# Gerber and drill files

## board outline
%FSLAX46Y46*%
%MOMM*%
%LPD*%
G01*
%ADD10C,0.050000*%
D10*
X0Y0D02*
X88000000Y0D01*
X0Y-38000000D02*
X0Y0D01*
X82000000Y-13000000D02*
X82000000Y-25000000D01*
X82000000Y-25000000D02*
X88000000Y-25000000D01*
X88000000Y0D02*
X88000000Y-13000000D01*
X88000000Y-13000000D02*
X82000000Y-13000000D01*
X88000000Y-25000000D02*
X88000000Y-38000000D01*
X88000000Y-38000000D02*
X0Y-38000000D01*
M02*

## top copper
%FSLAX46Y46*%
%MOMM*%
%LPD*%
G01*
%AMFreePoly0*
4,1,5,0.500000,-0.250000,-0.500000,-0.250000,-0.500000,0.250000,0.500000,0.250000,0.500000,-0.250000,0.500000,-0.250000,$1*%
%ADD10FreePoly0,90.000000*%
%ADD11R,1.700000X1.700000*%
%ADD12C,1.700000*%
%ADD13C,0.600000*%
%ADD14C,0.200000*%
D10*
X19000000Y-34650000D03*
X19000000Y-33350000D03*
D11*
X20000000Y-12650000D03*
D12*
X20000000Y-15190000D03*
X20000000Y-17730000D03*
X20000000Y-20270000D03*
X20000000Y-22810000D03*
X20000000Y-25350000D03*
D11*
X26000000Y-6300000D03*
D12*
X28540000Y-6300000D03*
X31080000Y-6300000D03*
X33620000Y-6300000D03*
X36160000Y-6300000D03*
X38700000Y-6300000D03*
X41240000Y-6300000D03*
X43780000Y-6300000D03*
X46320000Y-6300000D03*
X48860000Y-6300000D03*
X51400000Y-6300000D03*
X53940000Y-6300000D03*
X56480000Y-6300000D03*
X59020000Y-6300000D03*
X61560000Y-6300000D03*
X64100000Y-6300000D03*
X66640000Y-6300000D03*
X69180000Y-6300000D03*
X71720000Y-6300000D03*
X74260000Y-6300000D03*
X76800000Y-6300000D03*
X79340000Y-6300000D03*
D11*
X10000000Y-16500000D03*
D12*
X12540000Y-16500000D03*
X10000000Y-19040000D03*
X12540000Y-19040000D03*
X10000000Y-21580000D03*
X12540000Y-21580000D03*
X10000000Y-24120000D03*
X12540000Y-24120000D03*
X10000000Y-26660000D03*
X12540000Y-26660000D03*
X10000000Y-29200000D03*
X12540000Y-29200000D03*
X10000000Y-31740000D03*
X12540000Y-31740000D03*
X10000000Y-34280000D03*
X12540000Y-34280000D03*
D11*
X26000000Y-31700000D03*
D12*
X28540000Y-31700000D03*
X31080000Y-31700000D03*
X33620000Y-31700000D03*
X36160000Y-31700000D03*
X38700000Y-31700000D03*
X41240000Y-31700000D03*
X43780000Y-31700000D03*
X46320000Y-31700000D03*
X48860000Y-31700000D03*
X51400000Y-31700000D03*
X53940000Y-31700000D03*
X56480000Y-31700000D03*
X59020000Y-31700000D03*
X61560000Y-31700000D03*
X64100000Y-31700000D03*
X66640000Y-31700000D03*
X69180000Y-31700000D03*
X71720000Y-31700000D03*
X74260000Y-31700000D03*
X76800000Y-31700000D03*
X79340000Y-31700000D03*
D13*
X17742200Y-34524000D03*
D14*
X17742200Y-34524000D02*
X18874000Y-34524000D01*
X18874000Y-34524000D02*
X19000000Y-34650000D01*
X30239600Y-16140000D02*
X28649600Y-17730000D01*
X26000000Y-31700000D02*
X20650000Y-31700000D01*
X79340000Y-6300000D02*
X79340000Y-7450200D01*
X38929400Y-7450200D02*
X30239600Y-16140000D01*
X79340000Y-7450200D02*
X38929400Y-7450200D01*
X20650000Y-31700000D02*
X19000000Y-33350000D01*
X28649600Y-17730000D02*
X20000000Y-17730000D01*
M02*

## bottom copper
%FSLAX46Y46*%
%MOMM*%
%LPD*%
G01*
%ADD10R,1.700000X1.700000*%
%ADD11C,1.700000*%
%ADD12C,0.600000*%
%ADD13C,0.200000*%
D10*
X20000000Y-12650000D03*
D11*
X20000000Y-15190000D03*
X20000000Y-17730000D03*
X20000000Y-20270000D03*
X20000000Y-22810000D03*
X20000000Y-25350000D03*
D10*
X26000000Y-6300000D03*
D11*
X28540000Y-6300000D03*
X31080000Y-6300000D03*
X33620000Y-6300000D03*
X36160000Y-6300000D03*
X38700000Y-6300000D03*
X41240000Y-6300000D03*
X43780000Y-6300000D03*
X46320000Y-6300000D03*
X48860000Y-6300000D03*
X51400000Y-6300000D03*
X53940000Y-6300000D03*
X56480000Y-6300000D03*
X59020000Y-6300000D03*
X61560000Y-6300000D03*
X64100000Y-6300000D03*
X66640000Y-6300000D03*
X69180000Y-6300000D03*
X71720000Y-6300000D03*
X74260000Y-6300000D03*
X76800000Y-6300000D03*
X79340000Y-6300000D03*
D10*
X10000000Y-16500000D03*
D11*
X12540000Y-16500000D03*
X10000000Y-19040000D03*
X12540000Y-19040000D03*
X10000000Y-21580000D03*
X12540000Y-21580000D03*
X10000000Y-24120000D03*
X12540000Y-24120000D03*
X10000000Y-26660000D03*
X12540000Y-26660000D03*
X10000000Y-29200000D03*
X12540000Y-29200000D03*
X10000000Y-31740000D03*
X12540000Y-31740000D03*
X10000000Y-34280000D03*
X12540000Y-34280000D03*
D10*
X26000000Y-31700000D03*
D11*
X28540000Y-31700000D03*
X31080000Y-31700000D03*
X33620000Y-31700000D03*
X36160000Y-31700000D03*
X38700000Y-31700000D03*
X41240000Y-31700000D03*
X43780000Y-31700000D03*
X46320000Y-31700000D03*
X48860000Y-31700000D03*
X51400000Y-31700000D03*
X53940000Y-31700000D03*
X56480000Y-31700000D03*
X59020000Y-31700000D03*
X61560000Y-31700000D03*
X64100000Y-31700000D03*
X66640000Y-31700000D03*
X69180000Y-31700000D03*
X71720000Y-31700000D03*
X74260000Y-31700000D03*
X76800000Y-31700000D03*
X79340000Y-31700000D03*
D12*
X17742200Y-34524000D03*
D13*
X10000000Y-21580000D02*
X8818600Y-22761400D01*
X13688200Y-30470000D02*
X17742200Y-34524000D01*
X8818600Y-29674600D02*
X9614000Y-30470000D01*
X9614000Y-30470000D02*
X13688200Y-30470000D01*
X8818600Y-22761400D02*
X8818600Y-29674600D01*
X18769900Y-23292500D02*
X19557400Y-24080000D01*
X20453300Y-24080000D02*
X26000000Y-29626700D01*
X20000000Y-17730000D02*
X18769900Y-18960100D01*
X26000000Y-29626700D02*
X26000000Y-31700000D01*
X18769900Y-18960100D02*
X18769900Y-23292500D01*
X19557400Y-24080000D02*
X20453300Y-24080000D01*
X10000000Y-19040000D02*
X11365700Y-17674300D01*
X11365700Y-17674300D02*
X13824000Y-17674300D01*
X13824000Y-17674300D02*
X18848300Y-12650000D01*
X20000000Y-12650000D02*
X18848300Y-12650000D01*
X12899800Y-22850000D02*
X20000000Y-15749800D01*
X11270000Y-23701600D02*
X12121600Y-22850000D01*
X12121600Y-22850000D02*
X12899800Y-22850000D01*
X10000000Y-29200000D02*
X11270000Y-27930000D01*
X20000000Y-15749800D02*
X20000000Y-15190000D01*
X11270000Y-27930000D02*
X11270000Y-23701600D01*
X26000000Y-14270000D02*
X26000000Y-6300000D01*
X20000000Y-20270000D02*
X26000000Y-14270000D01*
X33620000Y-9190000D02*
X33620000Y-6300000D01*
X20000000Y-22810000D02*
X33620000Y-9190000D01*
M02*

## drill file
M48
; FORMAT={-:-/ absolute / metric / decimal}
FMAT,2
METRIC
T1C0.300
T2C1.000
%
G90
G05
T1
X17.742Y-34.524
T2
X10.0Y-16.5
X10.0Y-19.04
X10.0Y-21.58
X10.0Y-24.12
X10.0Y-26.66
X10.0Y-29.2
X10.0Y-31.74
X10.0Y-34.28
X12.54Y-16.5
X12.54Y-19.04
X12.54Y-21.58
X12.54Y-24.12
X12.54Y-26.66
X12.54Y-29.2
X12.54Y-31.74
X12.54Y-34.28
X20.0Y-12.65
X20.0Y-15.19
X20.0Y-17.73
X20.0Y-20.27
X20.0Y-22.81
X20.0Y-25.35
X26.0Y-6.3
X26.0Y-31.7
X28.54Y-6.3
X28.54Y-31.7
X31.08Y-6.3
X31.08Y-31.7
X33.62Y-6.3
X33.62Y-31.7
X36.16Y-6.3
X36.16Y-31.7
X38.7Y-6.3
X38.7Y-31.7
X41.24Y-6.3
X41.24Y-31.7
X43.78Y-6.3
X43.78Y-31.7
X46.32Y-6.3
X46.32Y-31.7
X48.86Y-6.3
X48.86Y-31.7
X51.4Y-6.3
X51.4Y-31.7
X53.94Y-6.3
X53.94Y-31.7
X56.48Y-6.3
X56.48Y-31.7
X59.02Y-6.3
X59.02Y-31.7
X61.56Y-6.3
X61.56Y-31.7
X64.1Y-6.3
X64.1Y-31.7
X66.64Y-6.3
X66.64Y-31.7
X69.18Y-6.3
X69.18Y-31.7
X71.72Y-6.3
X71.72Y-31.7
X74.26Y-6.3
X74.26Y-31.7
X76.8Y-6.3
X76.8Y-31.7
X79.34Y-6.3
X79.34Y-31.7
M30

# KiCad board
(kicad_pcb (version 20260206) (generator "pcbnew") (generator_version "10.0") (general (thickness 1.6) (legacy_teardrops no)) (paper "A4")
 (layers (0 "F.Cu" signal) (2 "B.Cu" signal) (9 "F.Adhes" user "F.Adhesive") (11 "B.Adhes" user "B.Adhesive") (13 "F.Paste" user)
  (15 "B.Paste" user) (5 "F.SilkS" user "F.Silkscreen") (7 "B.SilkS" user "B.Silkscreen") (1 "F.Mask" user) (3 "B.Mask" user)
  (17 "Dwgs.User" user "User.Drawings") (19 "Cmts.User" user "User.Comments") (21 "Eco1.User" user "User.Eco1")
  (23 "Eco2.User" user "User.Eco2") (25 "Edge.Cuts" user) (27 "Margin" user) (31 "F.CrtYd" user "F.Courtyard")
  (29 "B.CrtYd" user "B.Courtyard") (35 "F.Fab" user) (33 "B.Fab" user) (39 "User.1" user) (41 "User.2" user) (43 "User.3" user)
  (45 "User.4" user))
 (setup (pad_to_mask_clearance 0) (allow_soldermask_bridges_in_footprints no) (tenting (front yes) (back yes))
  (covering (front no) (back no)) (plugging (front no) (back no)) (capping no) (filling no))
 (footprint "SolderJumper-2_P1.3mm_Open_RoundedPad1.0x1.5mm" (layer "F.Cu") (at 19 34 90)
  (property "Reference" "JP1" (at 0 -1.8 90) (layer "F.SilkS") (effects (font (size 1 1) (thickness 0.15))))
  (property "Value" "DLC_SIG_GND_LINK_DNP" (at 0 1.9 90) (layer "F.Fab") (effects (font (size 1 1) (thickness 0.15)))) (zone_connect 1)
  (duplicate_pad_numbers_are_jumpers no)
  (pad "1" smd custom (at -0.65 0 90) (size 1 0.5) (layers "F.Cu" "F.Mask") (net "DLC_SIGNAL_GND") (zone_connect 2)
   (thermal_bridge_angle 45) (options (clearance outline) (anchor rect)) (primitives))
  (pad "2" smd custom (at 0.65 0 90) (size 1 0.5) (layers "F.Cu" "F.Mask") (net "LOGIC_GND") (zone_connect 2) (thermal_bridge_angle 45)
   (options (clearance outline) (anchor rect)) (primitives)))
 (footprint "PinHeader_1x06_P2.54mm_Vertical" (layer "F.Cu") (at 20 12.65)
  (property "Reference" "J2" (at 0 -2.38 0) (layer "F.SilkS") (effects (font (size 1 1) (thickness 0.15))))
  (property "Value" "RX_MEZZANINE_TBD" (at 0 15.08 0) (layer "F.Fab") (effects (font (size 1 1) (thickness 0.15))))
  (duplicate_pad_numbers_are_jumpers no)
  (pad "1" thru_hole rect (at 0 0) (size 1.7 1.7) (drill 1) (layers "*.Cu" "*.Mask") (remove_unused_layers no) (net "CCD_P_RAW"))
  (pad "2" thru_hole circle (at 0 2.54) (size 1.7 1.7) (drill 1) (layers "*.Cu" "*.Mask") (remove_unused_layers no) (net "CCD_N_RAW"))
  (pad "3" thru_hole circle (at 0 5.08) (size 1.7 1.7) (drill 1) (layers "*.Cu" "*.Mask") (remove_unused_layers no) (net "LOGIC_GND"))
  (pad "4" thru_hole circle (at 0 7.62) (size 1.7 1.7) (drill 1) (layers "*.Cu" "*.Mask") (remove_unused_layers no) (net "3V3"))
  (pad "5" thru_hole circle (at 0 10.16) (size 1.7 1.7) (drill 1) (layers "*.Cu" "*.Mask") (remove_unused_layers no) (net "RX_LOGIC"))
  (pad "6" thru_hole circle (at 0 12.7) (size 1.7 1.7) (drill 1) (layers "*.Cu" "*.Mask") (remove_unused_layers no)))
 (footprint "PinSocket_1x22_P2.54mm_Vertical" (layer "F.Cu") (at 26 6.3 90)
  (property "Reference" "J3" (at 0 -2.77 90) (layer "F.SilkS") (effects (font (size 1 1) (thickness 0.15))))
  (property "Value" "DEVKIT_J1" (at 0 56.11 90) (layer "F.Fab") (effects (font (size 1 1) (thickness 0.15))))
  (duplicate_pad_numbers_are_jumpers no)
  (pad "1" thru_hole rect (at 0 0 90) (size 1.7 1.7) (drill 1) (layers "*.Cu" "*.Mask") (remove_unused_layers no) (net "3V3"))
  (pad "2" thru_hole circle (at 0 2.54 90) (size 1.7 1.7) (drill 1) (layers "*.Cu" "*.Mask") (remove_unused_layers no))
  (pad "3" thru_hole circle (at 0 5.08 90) (size 1.7 1.7) (drill 1) (layers "*.Cu" "*.Mask") (remove_unused_layers no))
  (pad "4" thru_hole circle (at 0 7.62 90) (size 1.7 1.7) (drill 1) (layers "*.Cu" "*.Mask") (remove_unused_layers no) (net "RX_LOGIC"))
  (pad "5" thru_hole circle (at 0 10.16 90) (size 1.7 1.7) (drill 1) (layers "*.Cu" "*.Mask") (remove_unused_layers no))
  (pad "6" thru_hole circle (at 0 12.7 90) (size 1.7 1.7) (drill 1) (layers "*.Cu" "*.Mask") (remove_unused_layers no))
  (pad "7" thru_hole circle (at 0 15.24 90) (size 1.7 1.7) (drill 1) (layers "*.Cu" "*.Mask") (remove_unused_layers no))
  (pad "8" thru_hole circle (at 0 17.78 90) (size 1.7 1.7) (drill 1) (layers "*.Cu" "*.Mask") (remove_unused_layers no))
  (pad "9" thru_hole circle (at 0 20.32 90) (size 1.7 1.7) (drill 1) (layers "*.Cu" "*.Mask") (remove_unused_layers no))
  (pad "10" thru_hole circle (at 0 22.86 90) (size 1.7 1.7) (drill 1) (layers "*.Cu" "*.Mask") (remove_unused_layers no))
  (pad "11" thru_hole circle (at 0 25.4 90) (size 1.7 1.7) (drill 1) (layers "*.Cu" "*.Mask") (remove_unused_layers no))
  (pad "12" thru_hole circle (at 0 27.94 90) (size 1.7 1.7) (drill 1) (layers "*.Cu" "*.Mask") (remove_unused_layers no))
  (pad "13" thru_hole circle (at 0 30.48 90) (size 1.7 1.7) (drill 1) (layers "*.Cu" "*.Mask") (remove_unused_layers no))
  (pad "14" thru_hole circle (at 0 33.02 90) (size 1.7 1.7) (drill 1) (layers "*.Cu" "*.Mask") (remove_unused_layers no))
  (pad "15" thru_hole circle (at 0 35.56 90) (size 1.7 1.7) (drill 1) (layers "*.Cu" "*.Mask") (remove_unused_layers no))
  (pad "16" thru_hole circle (at 0 38.1 90) (size 1.7 1.7) (drill 1) (layers "*.Cu" "*.Mask") (remove_unused_layers no))
  (pad "17" thru_hole circle (at 0 40.64 90) (size 1.7 1.7) (drill 1) (layers "*.Cu" "*.Mask") (remove_unused_layers no))
  (pad "18" thru_hole circle (at 0 43.18 90) (size 1.7 1.7) (drill 1) (layers "*.Cu" "*.Mask") (remove_unused_layers no))
  (pad "19" thru_hole circle (at 0 45.72 90) (size 1.7 1.7) (drill 1) (layers "*.Cu" "*.Mask") (remove_unused_layers no))
  (pad "20" thru_hole circle (at 0 48.26 90) (size 1.7 1.7) (drill 1) (layers "*.Cu" "*.Mask") (remove_unused_layers no))
  (pad "21" thru_hole circle (at 0 50.8 90) (size 1.7 1.7) (drill 1) (layers "*.Cu" "*.Mask") (remove_unused_layers no))
  (pad "22" thru_hole circle (at 0 53.34 90) (size 1.7 1.7) (drill 1) (layers "*.Cu" "*.Mask") (remove_unused_layers no) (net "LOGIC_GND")))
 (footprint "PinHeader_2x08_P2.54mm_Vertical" (layer "F.Cu") (at 10 16.5)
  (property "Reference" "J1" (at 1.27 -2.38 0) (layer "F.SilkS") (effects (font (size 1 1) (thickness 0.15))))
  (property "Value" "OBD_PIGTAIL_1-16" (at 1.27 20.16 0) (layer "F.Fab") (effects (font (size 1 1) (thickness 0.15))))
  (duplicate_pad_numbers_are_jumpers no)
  (pad "1" thru_hole rect (at 0 0) (size 1.7 1.7) (drill 1) (layers "*.Cu" "*.Mask") (remove_unused_layers no))
  (pad "2" thru_hole circle (at 2.54 0) (size 1.7 1.7) (drill 1) (layers "*.Cu" "*.Mask") (remove_unused_layers no))
  (pad "3" thru_hole circle (at 0 2.54) (size 1.7 1.7) (drill 1) (layers "*.Cu" "*.Mask") (remove_unused_layers no) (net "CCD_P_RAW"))
  (pad "4" thru_hole circle (at 2.54 2.54) (size 1.7 1.7) (drill 1) (layers "*.Cu" "*.Mask") (remove_unused_layers no)
   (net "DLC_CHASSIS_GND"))
  (pad "5" thru_hole circle (at 0 5.08) (size 1.7 1.7) (drill 1) (layers "*.Cu" "*.Mask") (remove_unused_layers no) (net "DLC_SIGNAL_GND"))
  (pad "6" thru_hole circle (at 2.54 5.08) (size 1.7 1.7) (drill 1) (layers "*.Cu" "*.Mask") (remove_unused_layers no))
  (pad "7" thru_hole circle (at 0 7.62) (size 1.7 1.7) (drill 1) (layers "*.Cu" "*.Mask") (remove_unused_layers no))
  (pad "8" thru_hole circle (at 2.54 7.62) (size 1.7 1.7) (drill 1) (layers "*.Cu" "*.Mask") (remove_unused_layers no))
  (pad "9" thru_hole circle (at 0 10.16) (size 1.7 1.7) (drill 1) (layers "*.Cu" "*.Mask") (remove_unused_layers no))
  (pad "10" thru_hole circle (at 2.54 10.16) (size 1.7 1.7) (drill 1) (layers "*.Cu" "*.Mask") (remove_unused_layers no))
  (pad "11" thru_hole circle (at 0 12.7) (size 1.7 1.7) (drill 1) (layers "*.Cu" "*.Mask") (remove_unused_layers no) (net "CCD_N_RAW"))
  (pad "12" thru_hole circle (at 2.54 12.7) (size 1.7 1.7) (drill 1) (layers "*.Cu" "*.Mask") (remove_unused_layers no))
  (pad "13" thru_hole circle (at 0 15.24) (size 1.7 1.7) (drill 1) (layers "*.Cu" "*.Mask") (remove_unused_layers no))
  (pad "14" thru_hole circle (at 2.54 15.24) (size 1.7 1.7) (drill 1) (layers "*.Cu" "*.Mask") (remove_unused_layers no))
  (pad "15" thru_hole circle (at 0 17.78) (size 1.7 1.7) (drill 1) (layers "*.Cu" "*.Mask") (remove_unused_layers no))
  (pad "16" thru_hole circle (at 2.54 17.78) (size 1.7 1.7) (drill 1) (layers "*.Cu" "*.Mask") (remove_unused_layers no)))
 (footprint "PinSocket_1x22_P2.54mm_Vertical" (layer "F.Cu") (at 26 31.7 90)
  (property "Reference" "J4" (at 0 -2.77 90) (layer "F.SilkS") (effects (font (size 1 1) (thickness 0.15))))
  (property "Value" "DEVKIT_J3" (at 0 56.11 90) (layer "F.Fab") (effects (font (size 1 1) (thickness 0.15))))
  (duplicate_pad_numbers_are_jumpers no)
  (pad "1" thru_hole rect (at 0 0 90) (size 1.7 1.7) (drill 1) (layers "*.Cu" "*.Mask") (remove_unused_layers no) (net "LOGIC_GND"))
  (pad "2" thru_hole circle (at 0 2.54 90) (size 1.7 1.7) (drill 1) (layers "*.Cu" "*.Mask") (remove_unused_layers no))
  (pad "3" thru_hole circle (at 0 5.08 90) (size 1.7 1.7) (drill 1) (layers "*.Cu" "*.Mask") (remove_unused_layers no))
  (pad "4" thru_hole circle (at 0 7.62 90) (size 1.7 1.7) (drill 1) (layers "*.Cu" "*.Mask") (remove_unused_layers no))
  (pad "5" thru_hole circle (at 0 10.16 90) (size 1.7 1.7) (drill 1) (layers "*.Cu" "*.Mask") (remove_unused_layers no))
  (pad "6" thru_hole circle (at 0 12.7 90) (size 1.7 1.7) (drill 1) (layers "*.Cu" "*.Mask") (remove_unused_layers no))
  (pad "7" thru_hole circle (at 0 15.24 90) (size 1.7 1.7) (drill 1) (layers "*.Cu" "*.Mask") (remove_unused_layers no))
  (pad "8" thru_hole circle (at 0 17.78 90) (size 1.7 1.7) (drill 1) (layers "*.Cu" "*.Mask") (remove_unused_layers no))
  (pad "9" thru_hole circle (at 0 20.32 90) (size 1.7 1.7) (drill 1) (layers "*.Cu" "*.Mask") (remove_unused_layers no))
  (pad "10" thru_hole circle (at 0 22.86 90) (size 1.7 1.7) (drill 1) (layers "*.Cu" "*.Mask") (remove_unused_layers no))
  (pad "11" thru_hole circle (at 0 25.4 90) (size 1.7 1.7) (drill 1) (layers "*.Cu" "*.Mask") (remove_unused_layers no))
  (pad "12" thru_hole circle (at 0 27.94 90) (size 1.7 1.7) (drill 1) (layers "*.Cu" "*.Mask") (remove_unused_layers no))
  (pad "13" thru_hole circle (at 0 30.48 90) (size 1.7 1.7) (drill 1) (layers "*.Cu" "*.Mask") (remove_unused_layers no))
  (pad "14" thru_hole circle (at 0 33.02 90) (size 1.7 1.7) (drill 1) (layers "*.Cu" "*.Mask") (remove_unused_layers no))
  (pad "15" thru_hole circle (at 0 35.56 90) (size 1.7 1.7) (drill 1) (layers "*.Cu" "*.Mask") (remove_unused_layers no))
  (pad "16" thru_hole circle (at 0 38.1 90) (size 1.7 1.7) (drill 1) (layers "*.Cu" "*.Mask") (remove_unused_layers no))
  (pad "17" thru_hole circle (at 0 40.64 90) (size 1.7 1.7) (drill 1) (layers "*.Cu" "*.Mask") (remove_unused_layers no))
  (pad "18" thru_hole circle (at 0 43.18 90) (size 1.7 1.7) (drill 1) (layers "*.Cu" "*.Mask") (remove_unused_layers no))
  (pad "19" thru_hole circle (at 0 45.72 90) (size 1.7 1.7) (drill 1) (layers "*.Cu" "*.Mask") (remove_unused_layers no))
  (pad "20" thru_hole circle (at 0 48.26 90) (size 1.7 1.7) (drill 1) (layers "*.Cu" "*.Mask") (remove_unused_layers no))
  (pad "21" thru_hole circle (at 0 50.8 90) (size 1.7 1.7) (drill 1) (layers "*.Cu" "*.Mask") (remove_unused_layers no))
  (pad "22" thru_hole circle (at 0 53.34 90) (size 1.7 1.7) (drill 1) (layers "*.Cu" "*.Mask") (remove_unused_layers no)))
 (gr_line (start 0 0) (end 88 0) (stroke (width 0.05) (type default)) (layer "Edge.Cuts"))
 (gr_line (start 0 38) (end 0 0) (stroke (width 0.05) (type default)) (layer "Edge.Cuts"))
 (gr_line (start 82 13) (end 82 25) (stroke (width 0.05) (type default)) (layer "Edge.Cuts"))
 (gr_line (start 82 25) (end 88 25) (stroke (width 0.05) (type default)) (layer "Edge.Cuts"))
 (gr_line (start 88 0) (end 88 13) (stroke (width 0.05) (type default)) (layer "Edge.Cuts"))
 (gr_line (start 88 13) (end 82 13) (stroke (width 0.05) (type default)) (layer "Edge.Cuts"))
 (gr_line (start 88 25) (end 88 38) (stroke (width 0.05) (type default)) (layer "Edge.Cuts"))
 (gr_line (start 88 38) (end 0 38) (stroke (width 0.05) (type default)) (layer "Edge.Cuts"))
 (segment (start 17.7422 34.524) (end 18.874 34.524) (width 0.2) (layer "F.Cu") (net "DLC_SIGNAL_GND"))
 (segment (start 18.874 34.524) (end 19 34.65) (width 0.2) (layer "F.Cu") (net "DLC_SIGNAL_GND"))
 (via (at 17.7422 34.524) (size 0.6) (drill 0.3) (layers "F.Cu" "B.Cu") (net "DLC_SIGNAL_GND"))
 (segment (start 10 21.58) (end 8.8186 22.7614) (width 0.2) (layer "B.Cu") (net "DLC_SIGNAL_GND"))
 (segment (start 13.6882 30.47) (end 17.7422 34.524) (width 0.2) (layer "B.Cu") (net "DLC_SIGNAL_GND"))
 (segment (start 8.8186 29.6746) (end 9.614 30.47) (width 0.2) (layer "B.Cu") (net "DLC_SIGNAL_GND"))
 (segment (start 9.614 30.47) (end 13.6882 30.47) (width 0.2) (layer "B.Cu") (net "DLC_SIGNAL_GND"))
 (segment (start 8.8186 22.7614) (end 8.8186 29.6746) (width 0.2) (layer "B.Cu") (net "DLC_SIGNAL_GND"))
 (segment (start 30.2396 16.14) (end 28.6496 17.73) (width 0.2) (layer "F.Cu") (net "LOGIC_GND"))
 (segment (start 26 31.7) (end 20.65 31.7) (width 0.2) (layer "F.Cu") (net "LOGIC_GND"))
 (segment (start 79.34 6.3) (end 79.34 7.4502) (width 0.2) (layer "F.Cu") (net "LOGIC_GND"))
 (segment (start 38.9294 7.4502) (end 30.2396 16.14) (width 0.2) (layer "F.Cu") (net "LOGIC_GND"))
 (segment (start 79.34 7.4502) (end 38.9294 7.4502) (width 0.2) (layer "F.Cu") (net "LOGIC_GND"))
 (segment (start 20.65 31.7) (end 19 33.35) (width 0.2) (layer "F.Cu") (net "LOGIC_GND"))
 (segment (start 28.6496 17.73) (end 20 17.73) (width 0.2) (layer "F.Cu") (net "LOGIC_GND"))
 (segment (start 18.7699 23.2925) (end 19.5574 24.08) (width 0.2) (layer "B.Cu") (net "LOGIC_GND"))
 (segment (start 20.4533 24.08) (end 26 29.6267) (width 0.2) (layer "B.Cu") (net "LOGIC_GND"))
 (segment (start 20 17.73) (end 18.7699 18.9601) (width 0.2) (layer "B.Cu") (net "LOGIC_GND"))
 (segment (start 26 29.6267) (end 26 31.7) (width 0.2) (layer "B.Cu") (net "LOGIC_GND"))
 (segment (start 18.7699 18.9601) (end 18.7699 23.2925) (width 0.2) (layer "B.Cu") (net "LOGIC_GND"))
 (segment (start 19.5574 24.08) (end 20.4533 24.08) (width 0.2) (layer "B.Cu") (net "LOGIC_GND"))
 (segment (start 10 19.04) (end 11.3657 17.6743) (width 0.2) (layer "B.Cu") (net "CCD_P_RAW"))
 (segment (start 11.3657 17.6743) (end 13.824 17.6743) (width 0.2) (layer "B.Cu") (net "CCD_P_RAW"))
 (segment (start 13.824 17.6743) (end 18.8483 12.65) (width 0.2) (layer "B.Cu") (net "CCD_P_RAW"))
 (segment (start 20 12.65) (end 18.8483 12.65) (width 0.2) (layer "B.Cu") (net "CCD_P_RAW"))
 (segment (start 12.8998 22.85) (end 20 15.7498) (width 0.2) (layer "B.Cu") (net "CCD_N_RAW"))
 (segment (start 11.27 23.7016) (end 12.1216 22.85) (width 0.2) (layer "B.Cu") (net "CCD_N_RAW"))
 (segment (start 12.1216 22.85) (end 12.8998 22.85) (width 0.2) (layer "B.Cu") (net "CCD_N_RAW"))
 (segment (start 10 29.2) (end 11.27 27.93) (width 0.2) (layer "B.Cu") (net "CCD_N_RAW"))
 (segment (start 20 15.7498) (end 20 15.19) (width 0.2) (layer "B.Cu") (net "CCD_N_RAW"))
 (segment (start 11.27 27.93) (end 11.27 23.7016) (width 0.2) (layer "B.Cu") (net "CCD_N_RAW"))
 (segment (start 26 14.27) (end 26 6.3) (width 0.2) (layer "B.Cu") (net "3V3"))
 (segment (start 20 20.27) (end 26 14.27) (width 0.2) (layer "B.Cu") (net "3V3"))
 (segment (start 33.62 9.19) (end 33.62 6.3) (width 0.2) (layer "B.Cu") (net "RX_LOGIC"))
 (segment (start 20 22.81) (end 33.62 9.19) (width 0.2) (layer "B.Cu") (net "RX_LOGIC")))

